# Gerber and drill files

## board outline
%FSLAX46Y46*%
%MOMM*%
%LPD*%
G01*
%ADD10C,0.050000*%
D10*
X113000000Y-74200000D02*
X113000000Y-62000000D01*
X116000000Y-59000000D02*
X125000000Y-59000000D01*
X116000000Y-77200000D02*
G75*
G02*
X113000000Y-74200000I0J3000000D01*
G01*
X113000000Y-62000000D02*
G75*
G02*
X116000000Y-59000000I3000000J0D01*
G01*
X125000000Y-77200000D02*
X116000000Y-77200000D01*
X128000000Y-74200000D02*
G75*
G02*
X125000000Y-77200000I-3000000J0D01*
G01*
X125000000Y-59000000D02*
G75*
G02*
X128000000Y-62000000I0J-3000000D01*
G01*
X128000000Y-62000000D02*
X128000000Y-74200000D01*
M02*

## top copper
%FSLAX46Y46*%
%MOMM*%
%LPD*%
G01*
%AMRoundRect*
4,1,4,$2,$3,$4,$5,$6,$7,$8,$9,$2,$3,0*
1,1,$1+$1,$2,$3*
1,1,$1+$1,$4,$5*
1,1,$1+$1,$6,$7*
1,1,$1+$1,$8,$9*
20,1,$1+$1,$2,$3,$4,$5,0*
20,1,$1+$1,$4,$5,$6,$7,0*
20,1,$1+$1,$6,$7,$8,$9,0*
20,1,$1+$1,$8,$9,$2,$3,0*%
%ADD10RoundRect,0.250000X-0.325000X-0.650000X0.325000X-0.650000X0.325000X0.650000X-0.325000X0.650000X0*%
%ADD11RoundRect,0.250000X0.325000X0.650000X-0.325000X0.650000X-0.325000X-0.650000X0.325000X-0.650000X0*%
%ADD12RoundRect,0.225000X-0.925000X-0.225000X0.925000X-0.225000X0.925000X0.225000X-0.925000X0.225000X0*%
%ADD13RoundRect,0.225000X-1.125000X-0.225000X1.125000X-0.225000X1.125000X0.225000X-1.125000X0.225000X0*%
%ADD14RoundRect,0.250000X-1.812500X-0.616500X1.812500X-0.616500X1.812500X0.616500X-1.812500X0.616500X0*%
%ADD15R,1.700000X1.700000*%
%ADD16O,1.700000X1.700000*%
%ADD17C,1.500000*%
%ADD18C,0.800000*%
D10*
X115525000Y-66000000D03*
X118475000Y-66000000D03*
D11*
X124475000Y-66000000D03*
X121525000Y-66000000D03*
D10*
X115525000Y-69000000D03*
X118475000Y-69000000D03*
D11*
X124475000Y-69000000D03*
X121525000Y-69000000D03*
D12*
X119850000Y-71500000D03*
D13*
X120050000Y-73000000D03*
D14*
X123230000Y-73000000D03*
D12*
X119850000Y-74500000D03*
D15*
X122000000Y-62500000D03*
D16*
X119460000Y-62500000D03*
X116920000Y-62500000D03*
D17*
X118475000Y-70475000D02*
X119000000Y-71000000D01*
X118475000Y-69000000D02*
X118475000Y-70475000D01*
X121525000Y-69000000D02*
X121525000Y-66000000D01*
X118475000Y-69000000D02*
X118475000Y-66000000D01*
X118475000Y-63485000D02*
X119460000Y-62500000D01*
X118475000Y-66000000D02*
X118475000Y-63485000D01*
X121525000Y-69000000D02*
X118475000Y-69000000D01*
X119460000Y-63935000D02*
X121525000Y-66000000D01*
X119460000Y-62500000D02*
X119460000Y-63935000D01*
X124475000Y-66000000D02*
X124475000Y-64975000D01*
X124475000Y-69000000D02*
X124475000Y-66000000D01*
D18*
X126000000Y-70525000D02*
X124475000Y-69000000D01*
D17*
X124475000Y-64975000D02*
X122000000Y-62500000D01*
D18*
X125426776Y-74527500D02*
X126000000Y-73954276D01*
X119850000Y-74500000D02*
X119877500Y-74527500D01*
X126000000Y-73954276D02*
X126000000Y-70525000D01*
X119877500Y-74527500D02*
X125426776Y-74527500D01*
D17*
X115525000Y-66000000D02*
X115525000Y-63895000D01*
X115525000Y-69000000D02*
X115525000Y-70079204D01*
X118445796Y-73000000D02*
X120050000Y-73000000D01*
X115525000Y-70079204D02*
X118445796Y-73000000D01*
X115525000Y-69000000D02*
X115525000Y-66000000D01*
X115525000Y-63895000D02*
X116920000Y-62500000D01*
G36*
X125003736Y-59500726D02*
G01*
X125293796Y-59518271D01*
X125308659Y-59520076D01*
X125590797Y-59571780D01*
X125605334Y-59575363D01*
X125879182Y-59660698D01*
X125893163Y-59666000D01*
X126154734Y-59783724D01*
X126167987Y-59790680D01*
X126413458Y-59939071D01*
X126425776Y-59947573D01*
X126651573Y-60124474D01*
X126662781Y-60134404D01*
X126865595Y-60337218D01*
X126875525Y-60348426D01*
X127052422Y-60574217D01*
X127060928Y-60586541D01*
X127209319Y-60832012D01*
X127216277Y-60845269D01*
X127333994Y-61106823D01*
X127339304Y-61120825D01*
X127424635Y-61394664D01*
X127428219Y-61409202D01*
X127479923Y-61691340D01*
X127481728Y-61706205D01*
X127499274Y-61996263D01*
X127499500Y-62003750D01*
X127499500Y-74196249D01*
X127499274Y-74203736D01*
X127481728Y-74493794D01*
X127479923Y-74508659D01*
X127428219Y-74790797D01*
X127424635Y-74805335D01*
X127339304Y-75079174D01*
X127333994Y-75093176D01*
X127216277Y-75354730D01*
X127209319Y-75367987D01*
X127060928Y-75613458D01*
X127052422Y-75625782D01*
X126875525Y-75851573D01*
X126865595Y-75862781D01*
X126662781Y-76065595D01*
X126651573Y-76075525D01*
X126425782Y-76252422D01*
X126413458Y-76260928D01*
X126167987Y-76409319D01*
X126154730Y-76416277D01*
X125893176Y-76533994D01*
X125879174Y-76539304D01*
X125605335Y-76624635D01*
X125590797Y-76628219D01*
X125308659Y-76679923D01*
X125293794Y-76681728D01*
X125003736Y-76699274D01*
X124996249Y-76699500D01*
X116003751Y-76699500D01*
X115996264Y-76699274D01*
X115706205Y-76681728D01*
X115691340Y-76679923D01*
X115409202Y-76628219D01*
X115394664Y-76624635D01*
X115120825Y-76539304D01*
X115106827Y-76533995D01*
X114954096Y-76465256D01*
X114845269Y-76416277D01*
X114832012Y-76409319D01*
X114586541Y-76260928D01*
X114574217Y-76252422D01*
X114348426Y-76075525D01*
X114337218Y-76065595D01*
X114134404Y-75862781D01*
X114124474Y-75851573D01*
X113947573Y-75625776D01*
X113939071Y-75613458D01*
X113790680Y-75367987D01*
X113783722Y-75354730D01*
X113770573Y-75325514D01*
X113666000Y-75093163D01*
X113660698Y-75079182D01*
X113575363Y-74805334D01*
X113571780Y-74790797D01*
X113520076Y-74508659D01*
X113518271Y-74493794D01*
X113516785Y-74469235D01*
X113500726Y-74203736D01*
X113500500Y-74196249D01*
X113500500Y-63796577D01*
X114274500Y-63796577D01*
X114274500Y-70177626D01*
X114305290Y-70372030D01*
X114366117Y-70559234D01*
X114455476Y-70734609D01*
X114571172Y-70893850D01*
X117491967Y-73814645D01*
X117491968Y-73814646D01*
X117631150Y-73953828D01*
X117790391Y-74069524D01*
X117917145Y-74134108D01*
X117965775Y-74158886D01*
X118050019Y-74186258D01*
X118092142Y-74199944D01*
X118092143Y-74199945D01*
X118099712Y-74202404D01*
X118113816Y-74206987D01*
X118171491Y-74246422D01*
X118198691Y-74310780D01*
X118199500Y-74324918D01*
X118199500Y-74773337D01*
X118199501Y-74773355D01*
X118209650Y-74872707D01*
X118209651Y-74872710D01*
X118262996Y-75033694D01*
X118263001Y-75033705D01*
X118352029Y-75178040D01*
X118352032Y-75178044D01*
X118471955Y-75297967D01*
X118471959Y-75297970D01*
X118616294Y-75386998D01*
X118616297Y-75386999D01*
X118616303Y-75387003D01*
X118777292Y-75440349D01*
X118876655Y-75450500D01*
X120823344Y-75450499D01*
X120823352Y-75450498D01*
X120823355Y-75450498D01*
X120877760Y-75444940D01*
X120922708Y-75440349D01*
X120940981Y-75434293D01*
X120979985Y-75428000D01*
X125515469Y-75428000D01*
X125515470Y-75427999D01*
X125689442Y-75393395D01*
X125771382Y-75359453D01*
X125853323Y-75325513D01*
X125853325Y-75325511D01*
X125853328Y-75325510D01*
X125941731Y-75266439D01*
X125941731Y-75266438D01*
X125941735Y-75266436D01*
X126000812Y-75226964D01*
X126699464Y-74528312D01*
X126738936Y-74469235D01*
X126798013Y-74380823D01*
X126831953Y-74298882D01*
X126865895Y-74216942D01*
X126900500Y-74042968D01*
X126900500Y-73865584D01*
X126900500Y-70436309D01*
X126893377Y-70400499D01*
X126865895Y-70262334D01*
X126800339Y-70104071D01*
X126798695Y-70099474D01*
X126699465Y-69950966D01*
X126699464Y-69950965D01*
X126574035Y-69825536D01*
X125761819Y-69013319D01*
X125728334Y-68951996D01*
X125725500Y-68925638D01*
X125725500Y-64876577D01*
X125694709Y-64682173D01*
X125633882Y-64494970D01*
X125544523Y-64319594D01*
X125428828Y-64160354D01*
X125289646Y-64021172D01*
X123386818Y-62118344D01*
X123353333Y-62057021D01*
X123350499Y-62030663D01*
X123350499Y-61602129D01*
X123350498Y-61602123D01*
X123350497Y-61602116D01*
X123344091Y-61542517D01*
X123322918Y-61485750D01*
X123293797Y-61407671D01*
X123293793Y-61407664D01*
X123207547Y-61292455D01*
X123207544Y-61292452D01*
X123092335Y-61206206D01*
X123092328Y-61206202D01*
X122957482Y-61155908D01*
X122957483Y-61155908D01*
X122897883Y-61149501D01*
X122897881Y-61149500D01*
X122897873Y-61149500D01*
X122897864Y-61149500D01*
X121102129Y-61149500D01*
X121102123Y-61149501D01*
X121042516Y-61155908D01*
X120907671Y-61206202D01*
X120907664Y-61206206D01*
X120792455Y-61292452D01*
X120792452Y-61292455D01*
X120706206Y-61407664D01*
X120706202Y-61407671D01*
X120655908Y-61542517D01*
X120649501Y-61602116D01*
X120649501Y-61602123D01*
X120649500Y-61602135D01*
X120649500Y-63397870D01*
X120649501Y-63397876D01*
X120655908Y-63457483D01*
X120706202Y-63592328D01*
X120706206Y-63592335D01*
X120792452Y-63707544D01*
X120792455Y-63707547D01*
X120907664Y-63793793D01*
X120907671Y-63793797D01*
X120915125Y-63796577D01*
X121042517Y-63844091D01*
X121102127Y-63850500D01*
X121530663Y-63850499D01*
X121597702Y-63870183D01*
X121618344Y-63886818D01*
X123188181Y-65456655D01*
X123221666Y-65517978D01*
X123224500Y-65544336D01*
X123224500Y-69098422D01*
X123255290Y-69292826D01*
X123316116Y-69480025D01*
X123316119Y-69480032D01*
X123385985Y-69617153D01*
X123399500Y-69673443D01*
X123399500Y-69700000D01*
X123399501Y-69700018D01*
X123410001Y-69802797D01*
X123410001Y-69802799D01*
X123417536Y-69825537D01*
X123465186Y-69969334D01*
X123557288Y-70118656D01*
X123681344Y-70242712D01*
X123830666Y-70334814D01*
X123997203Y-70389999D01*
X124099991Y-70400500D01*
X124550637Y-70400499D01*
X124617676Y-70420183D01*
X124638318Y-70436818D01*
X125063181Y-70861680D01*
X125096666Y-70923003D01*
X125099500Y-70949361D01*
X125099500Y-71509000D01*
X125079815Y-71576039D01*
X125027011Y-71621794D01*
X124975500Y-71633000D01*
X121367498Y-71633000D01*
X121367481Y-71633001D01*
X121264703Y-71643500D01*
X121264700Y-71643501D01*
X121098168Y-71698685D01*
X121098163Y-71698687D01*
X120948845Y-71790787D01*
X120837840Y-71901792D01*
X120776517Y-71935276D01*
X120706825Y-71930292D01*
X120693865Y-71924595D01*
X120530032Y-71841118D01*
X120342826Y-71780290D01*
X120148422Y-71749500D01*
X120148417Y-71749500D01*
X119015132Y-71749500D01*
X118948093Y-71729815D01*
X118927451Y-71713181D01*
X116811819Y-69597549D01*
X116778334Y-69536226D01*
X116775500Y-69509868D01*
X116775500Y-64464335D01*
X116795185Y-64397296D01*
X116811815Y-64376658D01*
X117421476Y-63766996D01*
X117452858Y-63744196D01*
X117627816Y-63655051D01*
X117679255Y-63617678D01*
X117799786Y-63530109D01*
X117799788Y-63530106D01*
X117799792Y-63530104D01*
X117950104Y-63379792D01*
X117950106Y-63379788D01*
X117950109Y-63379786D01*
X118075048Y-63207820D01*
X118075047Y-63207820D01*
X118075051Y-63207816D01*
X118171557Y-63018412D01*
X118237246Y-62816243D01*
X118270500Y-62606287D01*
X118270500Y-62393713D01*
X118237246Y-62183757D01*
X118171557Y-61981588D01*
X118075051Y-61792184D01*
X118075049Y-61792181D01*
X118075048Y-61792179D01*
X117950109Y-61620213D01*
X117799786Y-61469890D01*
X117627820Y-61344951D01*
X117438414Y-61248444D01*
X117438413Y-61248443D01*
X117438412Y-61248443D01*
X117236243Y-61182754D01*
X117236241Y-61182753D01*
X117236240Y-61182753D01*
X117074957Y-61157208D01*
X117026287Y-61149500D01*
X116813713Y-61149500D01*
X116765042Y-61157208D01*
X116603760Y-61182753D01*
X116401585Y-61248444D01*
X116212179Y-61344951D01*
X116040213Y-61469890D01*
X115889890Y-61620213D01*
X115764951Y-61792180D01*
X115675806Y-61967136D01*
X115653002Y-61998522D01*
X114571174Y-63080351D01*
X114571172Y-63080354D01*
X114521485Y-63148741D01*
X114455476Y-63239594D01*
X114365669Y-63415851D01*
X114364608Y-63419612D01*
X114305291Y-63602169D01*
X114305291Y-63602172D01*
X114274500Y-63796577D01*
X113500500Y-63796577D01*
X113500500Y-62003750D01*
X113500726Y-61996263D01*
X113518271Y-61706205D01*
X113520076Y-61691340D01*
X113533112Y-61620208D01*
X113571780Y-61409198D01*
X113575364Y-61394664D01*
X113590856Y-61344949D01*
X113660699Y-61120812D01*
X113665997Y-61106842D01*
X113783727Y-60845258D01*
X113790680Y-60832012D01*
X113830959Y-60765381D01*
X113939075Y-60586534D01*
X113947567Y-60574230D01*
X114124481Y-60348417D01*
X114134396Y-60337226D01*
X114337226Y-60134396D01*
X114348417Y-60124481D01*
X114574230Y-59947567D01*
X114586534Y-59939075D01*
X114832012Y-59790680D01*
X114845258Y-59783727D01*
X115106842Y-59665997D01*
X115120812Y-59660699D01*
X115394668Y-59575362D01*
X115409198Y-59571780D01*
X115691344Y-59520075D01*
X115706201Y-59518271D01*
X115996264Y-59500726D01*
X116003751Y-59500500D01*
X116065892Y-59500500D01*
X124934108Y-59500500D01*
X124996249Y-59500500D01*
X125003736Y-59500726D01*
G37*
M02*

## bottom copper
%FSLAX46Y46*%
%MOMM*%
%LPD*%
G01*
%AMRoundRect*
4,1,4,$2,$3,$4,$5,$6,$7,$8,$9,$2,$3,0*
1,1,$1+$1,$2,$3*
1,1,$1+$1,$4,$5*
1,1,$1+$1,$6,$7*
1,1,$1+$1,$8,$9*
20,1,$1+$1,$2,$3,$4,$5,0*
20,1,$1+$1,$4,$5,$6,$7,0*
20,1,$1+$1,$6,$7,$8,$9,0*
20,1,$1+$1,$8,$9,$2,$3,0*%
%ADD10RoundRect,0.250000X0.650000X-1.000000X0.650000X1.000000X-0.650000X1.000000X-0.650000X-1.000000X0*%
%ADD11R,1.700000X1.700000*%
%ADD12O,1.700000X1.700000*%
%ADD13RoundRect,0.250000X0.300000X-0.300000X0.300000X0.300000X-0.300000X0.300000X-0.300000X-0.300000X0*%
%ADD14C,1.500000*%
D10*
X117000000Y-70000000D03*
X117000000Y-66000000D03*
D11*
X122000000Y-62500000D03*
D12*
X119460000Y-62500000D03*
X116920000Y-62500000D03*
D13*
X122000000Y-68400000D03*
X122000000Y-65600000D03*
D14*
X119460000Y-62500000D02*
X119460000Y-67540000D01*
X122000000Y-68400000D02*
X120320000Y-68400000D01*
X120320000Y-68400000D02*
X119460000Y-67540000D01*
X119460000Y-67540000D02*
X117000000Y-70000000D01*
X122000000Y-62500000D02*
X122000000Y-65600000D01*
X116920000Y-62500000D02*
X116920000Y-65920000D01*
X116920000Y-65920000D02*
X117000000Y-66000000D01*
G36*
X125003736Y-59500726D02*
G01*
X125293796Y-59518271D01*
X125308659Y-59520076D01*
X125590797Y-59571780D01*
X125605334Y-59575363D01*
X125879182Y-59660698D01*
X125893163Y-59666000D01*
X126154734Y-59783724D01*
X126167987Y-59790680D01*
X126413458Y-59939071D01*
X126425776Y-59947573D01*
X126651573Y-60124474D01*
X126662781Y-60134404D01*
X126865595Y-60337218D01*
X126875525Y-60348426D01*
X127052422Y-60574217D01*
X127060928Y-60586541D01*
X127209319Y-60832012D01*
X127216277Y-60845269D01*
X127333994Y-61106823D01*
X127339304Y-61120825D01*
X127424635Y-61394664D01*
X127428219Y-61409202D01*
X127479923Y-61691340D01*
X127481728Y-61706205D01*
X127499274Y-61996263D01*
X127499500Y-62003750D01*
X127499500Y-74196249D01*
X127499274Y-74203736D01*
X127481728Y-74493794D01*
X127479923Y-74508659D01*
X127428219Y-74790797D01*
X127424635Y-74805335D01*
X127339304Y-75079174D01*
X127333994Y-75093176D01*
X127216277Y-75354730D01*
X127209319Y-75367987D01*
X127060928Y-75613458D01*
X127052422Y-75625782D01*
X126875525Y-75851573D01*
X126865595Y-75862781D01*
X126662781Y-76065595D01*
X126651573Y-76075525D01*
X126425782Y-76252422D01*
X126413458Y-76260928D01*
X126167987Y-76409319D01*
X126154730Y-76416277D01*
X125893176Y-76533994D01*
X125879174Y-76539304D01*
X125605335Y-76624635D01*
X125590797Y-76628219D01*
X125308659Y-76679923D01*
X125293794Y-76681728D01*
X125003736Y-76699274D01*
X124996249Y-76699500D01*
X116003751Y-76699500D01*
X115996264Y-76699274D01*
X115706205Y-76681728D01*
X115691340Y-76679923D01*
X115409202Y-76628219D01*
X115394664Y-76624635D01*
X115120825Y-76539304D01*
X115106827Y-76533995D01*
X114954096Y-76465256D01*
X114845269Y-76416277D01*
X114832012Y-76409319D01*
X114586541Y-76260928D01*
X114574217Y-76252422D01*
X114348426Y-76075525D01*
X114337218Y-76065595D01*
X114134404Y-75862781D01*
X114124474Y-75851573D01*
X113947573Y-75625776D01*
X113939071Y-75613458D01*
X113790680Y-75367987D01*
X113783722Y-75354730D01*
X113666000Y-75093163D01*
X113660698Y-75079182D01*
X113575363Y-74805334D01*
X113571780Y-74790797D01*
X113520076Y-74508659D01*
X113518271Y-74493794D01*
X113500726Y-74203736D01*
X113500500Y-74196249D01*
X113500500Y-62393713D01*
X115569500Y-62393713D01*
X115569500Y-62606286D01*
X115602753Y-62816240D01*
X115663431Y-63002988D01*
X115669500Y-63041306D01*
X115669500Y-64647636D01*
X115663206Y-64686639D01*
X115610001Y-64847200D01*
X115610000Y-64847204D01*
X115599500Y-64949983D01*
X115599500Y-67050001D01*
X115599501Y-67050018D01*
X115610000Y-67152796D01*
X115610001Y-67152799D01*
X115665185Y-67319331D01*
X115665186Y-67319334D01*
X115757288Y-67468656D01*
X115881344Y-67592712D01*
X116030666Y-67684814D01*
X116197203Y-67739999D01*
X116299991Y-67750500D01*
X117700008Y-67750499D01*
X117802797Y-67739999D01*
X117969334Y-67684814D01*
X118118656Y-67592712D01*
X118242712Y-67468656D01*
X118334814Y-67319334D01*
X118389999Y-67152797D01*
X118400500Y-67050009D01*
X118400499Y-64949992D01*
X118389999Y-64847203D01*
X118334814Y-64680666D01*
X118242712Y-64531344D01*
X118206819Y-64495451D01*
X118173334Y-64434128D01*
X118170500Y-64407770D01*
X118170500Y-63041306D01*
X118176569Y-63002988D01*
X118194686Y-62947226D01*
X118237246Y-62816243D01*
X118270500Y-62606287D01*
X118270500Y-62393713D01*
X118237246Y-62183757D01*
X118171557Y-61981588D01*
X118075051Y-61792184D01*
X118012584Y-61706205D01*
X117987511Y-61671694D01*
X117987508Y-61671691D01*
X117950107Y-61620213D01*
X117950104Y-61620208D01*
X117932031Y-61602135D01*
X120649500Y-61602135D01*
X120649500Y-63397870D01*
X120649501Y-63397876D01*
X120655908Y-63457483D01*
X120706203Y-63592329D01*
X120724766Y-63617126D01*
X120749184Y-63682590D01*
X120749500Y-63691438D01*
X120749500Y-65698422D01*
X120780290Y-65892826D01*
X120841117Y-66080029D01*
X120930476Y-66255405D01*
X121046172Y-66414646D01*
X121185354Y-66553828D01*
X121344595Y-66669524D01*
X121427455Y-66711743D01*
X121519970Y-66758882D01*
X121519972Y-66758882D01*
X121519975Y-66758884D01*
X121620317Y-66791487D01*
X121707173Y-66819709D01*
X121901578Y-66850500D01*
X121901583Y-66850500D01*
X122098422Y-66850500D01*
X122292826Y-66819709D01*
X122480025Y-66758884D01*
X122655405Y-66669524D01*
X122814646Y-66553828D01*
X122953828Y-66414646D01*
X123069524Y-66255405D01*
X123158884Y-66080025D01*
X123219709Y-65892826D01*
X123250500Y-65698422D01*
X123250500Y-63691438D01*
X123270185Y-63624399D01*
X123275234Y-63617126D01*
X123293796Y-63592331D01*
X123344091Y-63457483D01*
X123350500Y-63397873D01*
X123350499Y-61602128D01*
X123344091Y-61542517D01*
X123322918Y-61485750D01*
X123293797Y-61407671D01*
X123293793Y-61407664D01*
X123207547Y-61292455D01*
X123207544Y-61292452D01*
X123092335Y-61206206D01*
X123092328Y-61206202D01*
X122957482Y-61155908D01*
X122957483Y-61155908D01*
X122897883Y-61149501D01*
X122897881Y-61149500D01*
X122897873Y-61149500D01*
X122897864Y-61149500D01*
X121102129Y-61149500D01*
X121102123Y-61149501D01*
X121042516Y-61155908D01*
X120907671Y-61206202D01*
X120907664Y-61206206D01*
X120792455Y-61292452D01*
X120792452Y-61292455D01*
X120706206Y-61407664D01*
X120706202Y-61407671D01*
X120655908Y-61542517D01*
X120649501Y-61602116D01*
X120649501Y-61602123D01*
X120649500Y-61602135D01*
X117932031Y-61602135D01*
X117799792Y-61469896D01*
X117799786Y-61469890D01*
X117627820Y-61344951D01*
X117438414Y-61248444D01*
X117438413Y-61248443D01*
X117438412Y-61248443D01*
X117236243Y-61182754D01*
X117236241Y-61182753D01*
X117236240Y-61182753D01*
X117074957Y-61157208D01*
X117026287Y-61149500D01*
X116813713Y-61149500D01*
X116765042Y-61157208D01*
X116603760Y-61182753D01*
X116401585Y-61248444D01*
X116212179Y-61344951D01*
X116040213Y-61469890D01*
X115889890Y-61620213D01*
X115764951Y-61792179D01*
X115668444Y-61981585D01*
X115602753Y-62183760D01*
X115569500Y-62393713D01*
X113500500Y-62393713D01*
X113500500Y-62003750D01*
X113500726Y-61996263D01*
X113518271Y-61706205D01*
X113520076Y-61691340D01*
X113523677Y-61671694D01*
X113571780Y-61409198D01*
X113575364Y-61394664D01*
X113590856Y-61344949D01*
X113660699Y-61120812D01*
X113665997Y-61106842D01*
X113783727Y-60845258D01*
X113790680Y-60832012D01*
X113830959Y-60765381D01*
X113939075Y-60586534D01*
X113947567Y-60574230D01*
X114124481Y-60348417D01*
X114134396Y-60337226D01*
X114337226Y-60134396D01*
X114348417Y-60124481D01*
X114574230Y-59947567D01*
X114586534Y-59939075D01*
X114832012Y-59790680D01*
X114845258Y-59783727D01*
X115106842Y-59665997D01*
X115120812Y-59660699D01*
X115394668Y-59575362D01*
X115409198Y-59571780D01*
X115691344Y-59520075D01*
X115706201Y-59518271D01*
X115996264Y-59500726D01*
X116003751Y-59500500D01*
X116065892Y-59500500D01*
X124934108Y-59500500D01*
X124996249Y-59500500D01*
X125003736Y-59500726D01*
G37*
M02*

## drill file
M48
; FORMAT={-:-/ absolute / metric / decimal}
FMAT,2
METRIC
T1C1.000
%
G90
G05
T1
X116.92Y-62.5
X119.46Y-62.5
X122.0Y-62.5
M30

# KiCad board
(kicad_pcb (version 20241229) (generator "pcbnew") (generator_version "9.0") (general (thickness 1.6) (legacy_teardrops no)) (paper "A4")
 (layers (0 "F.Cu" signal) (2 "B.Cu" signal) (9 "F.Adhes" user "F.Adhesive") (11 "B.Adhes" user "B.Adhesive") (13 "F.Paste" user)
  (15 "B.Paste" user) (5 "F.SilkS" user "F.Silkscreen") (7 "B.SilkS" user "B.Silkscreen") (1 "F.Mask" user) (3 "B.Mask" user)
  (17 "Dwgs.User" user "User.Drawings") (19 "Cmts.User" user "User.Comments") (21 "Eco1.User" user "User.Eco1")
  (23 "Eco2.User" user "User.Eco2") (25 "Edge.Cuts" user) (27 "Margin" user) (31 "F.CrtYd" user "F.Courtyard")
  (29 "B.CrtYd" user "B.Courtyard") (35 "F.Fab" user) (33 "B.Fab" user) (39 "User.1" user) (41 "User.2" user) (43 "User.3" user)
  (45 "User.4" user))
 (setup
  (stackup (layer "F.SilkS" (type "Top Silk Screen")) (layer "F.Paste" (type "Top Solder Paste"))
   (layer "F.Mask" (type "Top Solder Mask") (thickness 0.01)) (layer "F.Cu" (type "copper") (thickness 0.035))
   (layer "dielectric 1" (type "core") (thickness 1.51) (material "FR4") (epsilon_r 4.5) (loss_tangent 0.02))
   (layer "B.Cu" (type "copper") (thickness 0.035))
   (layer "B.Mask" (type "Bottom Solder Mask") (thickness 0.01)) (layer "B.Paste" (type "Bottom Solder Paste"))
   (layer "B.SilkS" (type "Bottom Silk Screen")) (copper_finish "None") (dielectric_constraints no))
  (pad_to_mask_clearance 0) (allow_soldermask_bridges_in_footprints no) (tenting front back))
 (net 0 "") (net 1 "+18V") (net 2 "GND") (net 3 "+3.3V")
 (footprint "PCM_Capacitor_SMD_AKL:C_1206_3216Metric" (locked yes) (layer "F.Cu") (at 117 66)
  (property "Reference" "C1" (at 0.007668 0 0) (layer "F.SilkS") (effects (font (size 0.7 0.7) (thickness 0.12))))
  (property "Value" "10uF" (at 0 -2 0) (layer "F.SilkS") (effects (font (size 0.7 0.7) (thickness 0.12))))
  (pad "1" smd roundrect (at -1.475 0) (size 1.15 1.8) (layers "F.Cu" "F.Mask" "F.Paste") (roundrect_rratio 0.217391) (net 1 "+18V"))
  (pad "2" smd roundrect (at 1.475 0) (size 1.15 1.8) (layers "F.Cu" "F.Mask" "F.Paste") (roundrect_rratio 0.217391) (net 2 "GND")))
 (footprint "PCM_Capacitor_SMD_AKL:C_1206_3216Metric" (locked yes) (layer "F.Cu") (at 123 66 180)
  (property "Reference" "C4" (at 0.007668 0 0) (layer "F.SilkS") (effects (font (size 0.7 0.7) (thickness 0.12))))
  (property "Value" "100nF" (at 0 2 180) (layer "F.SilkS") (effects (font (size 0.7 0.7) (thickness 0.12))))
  (pad "1" smd roundrect (at -1.475 0 180) (size 1.15 1.8) (layers "F.Cu" "F.Mask" "F.Paste") (roundrect_rratio 0.217391) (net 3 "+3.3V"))
  (pad "2" smd roundrect (at 1.475 0 180) (size 1.15 1.8) (layers "F.Cu" "F.Mask" "F.Paste") (roundrect_rratio 0.217391) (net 2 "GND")))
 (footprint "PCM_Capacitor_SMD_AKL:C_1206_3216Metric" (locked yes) (layer "F.Cu") (at 117 69)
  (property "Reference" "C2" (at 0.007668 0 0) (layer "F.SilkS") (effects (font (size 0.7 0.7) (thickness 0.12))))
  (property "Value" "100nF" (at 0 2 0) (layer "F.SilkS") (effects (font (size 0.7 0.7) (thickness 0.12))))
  (pad "1" smd roundrect (at -1.475 0) (size 1.15 1.8) (layers "F.Cu" "F.Mask" "F.Paste") (roundrect_rratio 0.217391) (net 1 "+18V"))
  (pad "2" smd roundrect (at 1.475 0) (size 1.15 1.8) (layers "F.Cu" "F.Mask" "F.Paste") (roundrect_rratio 0.217391) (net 2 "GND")))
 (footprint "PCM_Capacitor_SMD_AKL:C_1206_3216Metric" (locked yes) (layer "F.Cu") (at 123 69 180)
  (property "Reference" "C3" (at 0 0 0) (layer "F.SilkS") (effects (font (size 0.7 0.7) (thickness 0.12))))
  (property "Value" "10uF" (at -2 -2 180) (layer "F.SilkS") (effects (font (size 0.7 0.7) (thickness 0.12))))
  (pad "1" smd roundrect (at -1.475 0 180) (size 1.15 1.8) (layers "F.Cu" "F.Mask" "F.Paste") (roundrect_rratio 0.217391) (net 3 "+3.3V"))
  (pad "2" smd roundrect (at 1.475 0 180) (size 1.15 1.8) (layers "F.Cu" "F.Mask" "F.Paste") (roundrect_rratio 0.217391) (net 2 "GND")))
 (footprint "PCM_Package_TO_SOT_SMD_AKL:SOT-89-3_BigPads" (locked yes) (layer "F.Cu") (at 122 73)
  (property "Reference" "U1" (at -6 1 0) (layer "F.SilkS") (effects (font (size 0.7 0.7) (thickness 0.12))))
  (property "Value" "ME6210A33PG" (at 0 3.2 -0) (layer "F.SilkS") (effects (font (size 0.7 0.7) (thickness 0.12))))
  (pad "1" smd roundrect (at -2.15 -1.5) (size 2.3 0.9) (layers "F.Cu" "F.Mask" "F.Paste") (roundrect_rratio 0.25) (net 2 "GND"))
  (pad "2" smd roundrect (at -1.95 0) (size 2.7 0.9) (layers "F.Cu" "F.Mask" "F.Paste") (roundrect_rratio 0.25) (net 1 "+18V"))
  (pad "2" smd roundrect (at 1.23 0) (size 4.125 1.733) (layers "F.Cu" "F.Mask" "F.Paste") (roundrect_rratio 0.1442585113) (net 1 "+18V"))
  (pad "3" smd roundrect (at -2.15 1.5) (size 2.3 0.9) (layers "F.Cu" "F.Mask" "F.Paste") (roundrect_rratio 0.25) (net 3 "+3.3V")))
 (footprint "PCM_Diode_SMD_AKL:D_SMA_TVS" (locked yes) (layer "B.Cu") (at 117 68 90)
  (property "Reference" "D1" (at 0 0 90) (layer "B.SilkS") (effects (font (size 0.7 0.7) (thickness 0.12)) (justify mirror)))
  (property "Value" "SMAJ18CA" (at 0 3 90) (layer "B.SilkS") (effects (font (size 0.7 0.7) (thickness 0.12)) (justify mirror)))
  (pad "1" smd roundrect (at -2 0 90) (size 2.5 1.8) (layers "B.Cu" "B.Mask" "B.Paste") (roundrect_rratio 0.1388888889) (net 2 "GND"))
  (pad "2" smd roundrect (at 2 0 90) (size 2.5 1.8) (layers "B.Cu" "B.Mask" "B.Paste") (roundrect_rratio 0.1388888889) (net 1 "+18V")))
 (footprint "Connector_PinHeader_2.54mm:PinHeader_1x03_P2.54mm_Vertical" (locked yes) (layer "B.Cu") (at 122 62.5 90)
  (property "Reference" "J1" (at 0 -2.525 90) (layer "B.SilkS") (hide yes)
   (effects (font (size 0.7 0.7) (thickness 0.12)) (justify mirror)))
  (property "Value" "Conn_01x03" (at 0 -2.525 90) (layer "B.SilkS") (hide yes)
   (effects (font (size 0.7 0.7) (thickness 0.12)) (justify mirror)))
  (pad "1" thru_hole rect (at 0 0 90) (size 1.7 1.7) (drill 1) (layers "*.Cu" "*.Mask") (remove_unused_layers no) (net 3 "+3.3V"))
  (pad "2" thru_hole oval (at 0 -2.54 90) (size 1.7 1.7) (drill 1) (layers "*.Cu" "*.Mask") (remove_unused_layers no) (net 2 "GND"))
  (pad "3" thru_hole oval (at 0 -5.08 90) (size 1.7 1.7) (drill 1) (layers "*.Cu" "*.Mask") (remove_unused_layers no) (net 1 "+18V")))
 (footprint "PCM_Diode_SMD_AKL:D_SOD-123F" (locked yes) (layer "B.Cu") (at 122 67 90)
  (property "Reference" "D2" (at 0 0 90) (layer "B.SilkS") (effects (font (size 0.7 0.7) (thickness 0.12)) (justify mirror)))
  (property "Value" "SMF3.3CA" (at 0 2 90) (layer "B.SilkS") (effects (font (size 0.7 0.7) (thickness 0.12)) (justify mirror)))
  (pad "1" smd roundrect (at -1.4 0 90) (size 1.1 1.1) (layers "B.Cu" "B.Mask" "B.Paste") (roundrect_rratio 0.2272727273) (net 2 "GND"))
  (pad "2" smd roundrect (at 1.4 0 90) (size 1.1 1.1) (layers "B.Cu" "B.Mask" "B.Paste") (roundrect_rratio 0.2272727273) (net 3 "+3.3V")))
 (gr_line (start 113 74.2) (end 113 62) (stroke (width 0.05) (type default)) (locked yes) (layer "Edge.Cuts"))
 (gr_line (start 116 59) (end 125 59) (stroke (width 0.05) (type default)) (locked yes) (layer "Edge.Cuts"))
 (gr_arc (start 116 77.2) (mid 113.87868 76.32132) (end 113 74.2) (stroke (width 0.05) (type default)) (locked yes) (layer "Edge.Cuts"))
 (gr_arc (start 113 62) (mid 113.87868 59.87868) (end 116 59) (stroke (width 0.05) (type default)) (locked yes) (layer "Edge.Cuts"))
 (gr_line (start 125 77.2) (end 116 77.2) (stroke (width 0.05) (type default)) (locked yes) (layer "Edge.Cuts"))
 (gr_arc (start 128 74.2) (mid 127.12132 76.32132) (end 125 77.2) (stroke (width 0.05) (type default)) (locked yes) (layer "Edge.Cuts"))
 (gr_arc (start 125 59) (mid 127.12132 59.87868) (end 128 62) (stroke (width 0.05) (type default)) (locked yes) (layer "Edge.Cuts"))
 (gr_line (start 128 62) (end 128 74.2) (stroke (width 0.05) (type default)) (locked yes) (layer "Edge.Cuts"))
 (segment (start 118.475 70.475) (end 119 71) (width 1.5) (locked yes) (layer "F.Cu") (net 2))
 (segment (start 118.475 69) (end 118.475 70.475) (width 1.5) (locked yes) (layer "F.Cu") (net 2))
 (segment (start 121.525 69) (end 121.525 66) (width 1.5) (locked yes) (layer "F.Cu") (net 2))
 (segment (start 118.475 69) (end 118.475 66) (width 1.5) (locked yes) (layer "F.Cu") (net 2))
 (segment (start 118.475 63.485) (end 119.46 62.5) (width 1.5) (locked yes) (layer "F.Cu") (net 2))
 (segment (start 118.475 66) (end 118.475 63.485) (width 1.5) (locked yes) (layer "F.Cu") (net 2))
 (segment (start 121.525 69) (end 118.475 69) (width 1.5) (locked yes) (layer "F.Cu") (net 2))
 (segment (start 119.46 63.935) (end 121.525 66) (width 1.5) (locked yes) (layer "F.Cu") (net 2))
 (segment (start 119.46 62.5) (end 119.46 63.935) (width 1.5) (locked yes) (layer "F.Cu") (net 2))
 (segment (start 119.46 62.5) (end 119.46 67.54) (width 1.5) (locked yes) (layer "B.Cu") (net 2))
 (segment (start 122 68.4) (end 120.32 68.4) (width 1.5) (locked yes) (layer "B.Cu") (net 2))
 (segment (start 120.32 68.4) (end 119.46 67.54) (width 1.5) (locked yes) (layer "B.Cu") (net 2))
 (segment (start 119.46 67.54) (end 117 70) (width 1.5) (locked yes) (layer "B.Cu") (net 2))
 (segment (start 124.475 66) (end 124.475 64.975) (width 1.5) (locked yes) (layer "F.Cu") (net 3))
 (segment (start 124.475 69) (end 124.475 66) (width 1.5) (locked yes) (layer "F.Cu") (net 3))
 (segment (start 126 70.525) (end 124.475 69) (width 0.8) (locked yes) (layer "F.Cu") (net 3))
 (segment (start 124.475 64.975) (end 122 62.5) (width 1.5) (locked yes) (layer "F.Cu") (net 3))
 (segment (start 125.426776 74.5275) (end 126 73.954276) (width 0.8) (locked yes) (layer "F.Cu") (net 3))
 (segment (start 119.85 74.5) (end 119.8775 74.5275) (width 0.8) (locked yes) (layer "F.Cu") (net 3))
 (segment (start 126 73.954276) (end 126 70.525) (width 0.8) (locked yes) (layer "F.Cu") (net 3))
 (segment (start 119.8775 74.5275) (end 125.426776 74.5275) (width 0.8) (locked yes) (layer "F.Cu") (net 3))
 (segment (start 122 62.5) (end 122 65.6) (width 1.5) (locked yes) (layer "B.Cu") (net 3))
 (segment (start 115.525 66) (end 115.525 63.895) (width 1.5) (locked yes) (layer "F.Cu") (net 1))
 (segment (start 115.525 69) (end 115.525 70.079204) (width 1.5) (locked yes) (layer "F.Cu") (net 1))
 (segment (start 118.445796 73) (end 120.05 73) (width 1.5) (locked yes) (layer "F.Cu") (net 1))
 (segment (start 115.525 70.079204) (end 118.445796 73) (width 1.5) (locked yes) (layer "F.Cu") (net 1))
 (segment (start 115.525 69) (end 115.525 66) (width 1.5) (locked yes) (layer "F.Cu") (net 1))
 (segment (start 115.525 63.895) (end 116.92 62.5) (width 1.5) (locked yes) (layer "F.Cu") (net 1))
 (segment (start 116.92 62.5) (end 116.92 65.92) (width 1.5) (locked yes) (layer "B.Cu") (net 1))
 (segment (start 116.92 65.92) (end 117 66) (width 1.5) (locked yes) (layer "B.Cu") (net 1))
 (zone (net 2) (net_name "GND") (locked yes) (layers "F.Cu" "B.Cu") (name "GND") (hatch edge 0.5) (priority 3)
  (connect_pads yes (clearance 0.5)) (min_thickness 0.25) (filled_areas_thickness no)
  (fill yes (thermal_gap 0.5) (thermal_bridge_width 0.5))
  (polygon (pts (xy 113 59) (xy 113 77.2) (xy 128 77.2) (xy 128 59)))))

